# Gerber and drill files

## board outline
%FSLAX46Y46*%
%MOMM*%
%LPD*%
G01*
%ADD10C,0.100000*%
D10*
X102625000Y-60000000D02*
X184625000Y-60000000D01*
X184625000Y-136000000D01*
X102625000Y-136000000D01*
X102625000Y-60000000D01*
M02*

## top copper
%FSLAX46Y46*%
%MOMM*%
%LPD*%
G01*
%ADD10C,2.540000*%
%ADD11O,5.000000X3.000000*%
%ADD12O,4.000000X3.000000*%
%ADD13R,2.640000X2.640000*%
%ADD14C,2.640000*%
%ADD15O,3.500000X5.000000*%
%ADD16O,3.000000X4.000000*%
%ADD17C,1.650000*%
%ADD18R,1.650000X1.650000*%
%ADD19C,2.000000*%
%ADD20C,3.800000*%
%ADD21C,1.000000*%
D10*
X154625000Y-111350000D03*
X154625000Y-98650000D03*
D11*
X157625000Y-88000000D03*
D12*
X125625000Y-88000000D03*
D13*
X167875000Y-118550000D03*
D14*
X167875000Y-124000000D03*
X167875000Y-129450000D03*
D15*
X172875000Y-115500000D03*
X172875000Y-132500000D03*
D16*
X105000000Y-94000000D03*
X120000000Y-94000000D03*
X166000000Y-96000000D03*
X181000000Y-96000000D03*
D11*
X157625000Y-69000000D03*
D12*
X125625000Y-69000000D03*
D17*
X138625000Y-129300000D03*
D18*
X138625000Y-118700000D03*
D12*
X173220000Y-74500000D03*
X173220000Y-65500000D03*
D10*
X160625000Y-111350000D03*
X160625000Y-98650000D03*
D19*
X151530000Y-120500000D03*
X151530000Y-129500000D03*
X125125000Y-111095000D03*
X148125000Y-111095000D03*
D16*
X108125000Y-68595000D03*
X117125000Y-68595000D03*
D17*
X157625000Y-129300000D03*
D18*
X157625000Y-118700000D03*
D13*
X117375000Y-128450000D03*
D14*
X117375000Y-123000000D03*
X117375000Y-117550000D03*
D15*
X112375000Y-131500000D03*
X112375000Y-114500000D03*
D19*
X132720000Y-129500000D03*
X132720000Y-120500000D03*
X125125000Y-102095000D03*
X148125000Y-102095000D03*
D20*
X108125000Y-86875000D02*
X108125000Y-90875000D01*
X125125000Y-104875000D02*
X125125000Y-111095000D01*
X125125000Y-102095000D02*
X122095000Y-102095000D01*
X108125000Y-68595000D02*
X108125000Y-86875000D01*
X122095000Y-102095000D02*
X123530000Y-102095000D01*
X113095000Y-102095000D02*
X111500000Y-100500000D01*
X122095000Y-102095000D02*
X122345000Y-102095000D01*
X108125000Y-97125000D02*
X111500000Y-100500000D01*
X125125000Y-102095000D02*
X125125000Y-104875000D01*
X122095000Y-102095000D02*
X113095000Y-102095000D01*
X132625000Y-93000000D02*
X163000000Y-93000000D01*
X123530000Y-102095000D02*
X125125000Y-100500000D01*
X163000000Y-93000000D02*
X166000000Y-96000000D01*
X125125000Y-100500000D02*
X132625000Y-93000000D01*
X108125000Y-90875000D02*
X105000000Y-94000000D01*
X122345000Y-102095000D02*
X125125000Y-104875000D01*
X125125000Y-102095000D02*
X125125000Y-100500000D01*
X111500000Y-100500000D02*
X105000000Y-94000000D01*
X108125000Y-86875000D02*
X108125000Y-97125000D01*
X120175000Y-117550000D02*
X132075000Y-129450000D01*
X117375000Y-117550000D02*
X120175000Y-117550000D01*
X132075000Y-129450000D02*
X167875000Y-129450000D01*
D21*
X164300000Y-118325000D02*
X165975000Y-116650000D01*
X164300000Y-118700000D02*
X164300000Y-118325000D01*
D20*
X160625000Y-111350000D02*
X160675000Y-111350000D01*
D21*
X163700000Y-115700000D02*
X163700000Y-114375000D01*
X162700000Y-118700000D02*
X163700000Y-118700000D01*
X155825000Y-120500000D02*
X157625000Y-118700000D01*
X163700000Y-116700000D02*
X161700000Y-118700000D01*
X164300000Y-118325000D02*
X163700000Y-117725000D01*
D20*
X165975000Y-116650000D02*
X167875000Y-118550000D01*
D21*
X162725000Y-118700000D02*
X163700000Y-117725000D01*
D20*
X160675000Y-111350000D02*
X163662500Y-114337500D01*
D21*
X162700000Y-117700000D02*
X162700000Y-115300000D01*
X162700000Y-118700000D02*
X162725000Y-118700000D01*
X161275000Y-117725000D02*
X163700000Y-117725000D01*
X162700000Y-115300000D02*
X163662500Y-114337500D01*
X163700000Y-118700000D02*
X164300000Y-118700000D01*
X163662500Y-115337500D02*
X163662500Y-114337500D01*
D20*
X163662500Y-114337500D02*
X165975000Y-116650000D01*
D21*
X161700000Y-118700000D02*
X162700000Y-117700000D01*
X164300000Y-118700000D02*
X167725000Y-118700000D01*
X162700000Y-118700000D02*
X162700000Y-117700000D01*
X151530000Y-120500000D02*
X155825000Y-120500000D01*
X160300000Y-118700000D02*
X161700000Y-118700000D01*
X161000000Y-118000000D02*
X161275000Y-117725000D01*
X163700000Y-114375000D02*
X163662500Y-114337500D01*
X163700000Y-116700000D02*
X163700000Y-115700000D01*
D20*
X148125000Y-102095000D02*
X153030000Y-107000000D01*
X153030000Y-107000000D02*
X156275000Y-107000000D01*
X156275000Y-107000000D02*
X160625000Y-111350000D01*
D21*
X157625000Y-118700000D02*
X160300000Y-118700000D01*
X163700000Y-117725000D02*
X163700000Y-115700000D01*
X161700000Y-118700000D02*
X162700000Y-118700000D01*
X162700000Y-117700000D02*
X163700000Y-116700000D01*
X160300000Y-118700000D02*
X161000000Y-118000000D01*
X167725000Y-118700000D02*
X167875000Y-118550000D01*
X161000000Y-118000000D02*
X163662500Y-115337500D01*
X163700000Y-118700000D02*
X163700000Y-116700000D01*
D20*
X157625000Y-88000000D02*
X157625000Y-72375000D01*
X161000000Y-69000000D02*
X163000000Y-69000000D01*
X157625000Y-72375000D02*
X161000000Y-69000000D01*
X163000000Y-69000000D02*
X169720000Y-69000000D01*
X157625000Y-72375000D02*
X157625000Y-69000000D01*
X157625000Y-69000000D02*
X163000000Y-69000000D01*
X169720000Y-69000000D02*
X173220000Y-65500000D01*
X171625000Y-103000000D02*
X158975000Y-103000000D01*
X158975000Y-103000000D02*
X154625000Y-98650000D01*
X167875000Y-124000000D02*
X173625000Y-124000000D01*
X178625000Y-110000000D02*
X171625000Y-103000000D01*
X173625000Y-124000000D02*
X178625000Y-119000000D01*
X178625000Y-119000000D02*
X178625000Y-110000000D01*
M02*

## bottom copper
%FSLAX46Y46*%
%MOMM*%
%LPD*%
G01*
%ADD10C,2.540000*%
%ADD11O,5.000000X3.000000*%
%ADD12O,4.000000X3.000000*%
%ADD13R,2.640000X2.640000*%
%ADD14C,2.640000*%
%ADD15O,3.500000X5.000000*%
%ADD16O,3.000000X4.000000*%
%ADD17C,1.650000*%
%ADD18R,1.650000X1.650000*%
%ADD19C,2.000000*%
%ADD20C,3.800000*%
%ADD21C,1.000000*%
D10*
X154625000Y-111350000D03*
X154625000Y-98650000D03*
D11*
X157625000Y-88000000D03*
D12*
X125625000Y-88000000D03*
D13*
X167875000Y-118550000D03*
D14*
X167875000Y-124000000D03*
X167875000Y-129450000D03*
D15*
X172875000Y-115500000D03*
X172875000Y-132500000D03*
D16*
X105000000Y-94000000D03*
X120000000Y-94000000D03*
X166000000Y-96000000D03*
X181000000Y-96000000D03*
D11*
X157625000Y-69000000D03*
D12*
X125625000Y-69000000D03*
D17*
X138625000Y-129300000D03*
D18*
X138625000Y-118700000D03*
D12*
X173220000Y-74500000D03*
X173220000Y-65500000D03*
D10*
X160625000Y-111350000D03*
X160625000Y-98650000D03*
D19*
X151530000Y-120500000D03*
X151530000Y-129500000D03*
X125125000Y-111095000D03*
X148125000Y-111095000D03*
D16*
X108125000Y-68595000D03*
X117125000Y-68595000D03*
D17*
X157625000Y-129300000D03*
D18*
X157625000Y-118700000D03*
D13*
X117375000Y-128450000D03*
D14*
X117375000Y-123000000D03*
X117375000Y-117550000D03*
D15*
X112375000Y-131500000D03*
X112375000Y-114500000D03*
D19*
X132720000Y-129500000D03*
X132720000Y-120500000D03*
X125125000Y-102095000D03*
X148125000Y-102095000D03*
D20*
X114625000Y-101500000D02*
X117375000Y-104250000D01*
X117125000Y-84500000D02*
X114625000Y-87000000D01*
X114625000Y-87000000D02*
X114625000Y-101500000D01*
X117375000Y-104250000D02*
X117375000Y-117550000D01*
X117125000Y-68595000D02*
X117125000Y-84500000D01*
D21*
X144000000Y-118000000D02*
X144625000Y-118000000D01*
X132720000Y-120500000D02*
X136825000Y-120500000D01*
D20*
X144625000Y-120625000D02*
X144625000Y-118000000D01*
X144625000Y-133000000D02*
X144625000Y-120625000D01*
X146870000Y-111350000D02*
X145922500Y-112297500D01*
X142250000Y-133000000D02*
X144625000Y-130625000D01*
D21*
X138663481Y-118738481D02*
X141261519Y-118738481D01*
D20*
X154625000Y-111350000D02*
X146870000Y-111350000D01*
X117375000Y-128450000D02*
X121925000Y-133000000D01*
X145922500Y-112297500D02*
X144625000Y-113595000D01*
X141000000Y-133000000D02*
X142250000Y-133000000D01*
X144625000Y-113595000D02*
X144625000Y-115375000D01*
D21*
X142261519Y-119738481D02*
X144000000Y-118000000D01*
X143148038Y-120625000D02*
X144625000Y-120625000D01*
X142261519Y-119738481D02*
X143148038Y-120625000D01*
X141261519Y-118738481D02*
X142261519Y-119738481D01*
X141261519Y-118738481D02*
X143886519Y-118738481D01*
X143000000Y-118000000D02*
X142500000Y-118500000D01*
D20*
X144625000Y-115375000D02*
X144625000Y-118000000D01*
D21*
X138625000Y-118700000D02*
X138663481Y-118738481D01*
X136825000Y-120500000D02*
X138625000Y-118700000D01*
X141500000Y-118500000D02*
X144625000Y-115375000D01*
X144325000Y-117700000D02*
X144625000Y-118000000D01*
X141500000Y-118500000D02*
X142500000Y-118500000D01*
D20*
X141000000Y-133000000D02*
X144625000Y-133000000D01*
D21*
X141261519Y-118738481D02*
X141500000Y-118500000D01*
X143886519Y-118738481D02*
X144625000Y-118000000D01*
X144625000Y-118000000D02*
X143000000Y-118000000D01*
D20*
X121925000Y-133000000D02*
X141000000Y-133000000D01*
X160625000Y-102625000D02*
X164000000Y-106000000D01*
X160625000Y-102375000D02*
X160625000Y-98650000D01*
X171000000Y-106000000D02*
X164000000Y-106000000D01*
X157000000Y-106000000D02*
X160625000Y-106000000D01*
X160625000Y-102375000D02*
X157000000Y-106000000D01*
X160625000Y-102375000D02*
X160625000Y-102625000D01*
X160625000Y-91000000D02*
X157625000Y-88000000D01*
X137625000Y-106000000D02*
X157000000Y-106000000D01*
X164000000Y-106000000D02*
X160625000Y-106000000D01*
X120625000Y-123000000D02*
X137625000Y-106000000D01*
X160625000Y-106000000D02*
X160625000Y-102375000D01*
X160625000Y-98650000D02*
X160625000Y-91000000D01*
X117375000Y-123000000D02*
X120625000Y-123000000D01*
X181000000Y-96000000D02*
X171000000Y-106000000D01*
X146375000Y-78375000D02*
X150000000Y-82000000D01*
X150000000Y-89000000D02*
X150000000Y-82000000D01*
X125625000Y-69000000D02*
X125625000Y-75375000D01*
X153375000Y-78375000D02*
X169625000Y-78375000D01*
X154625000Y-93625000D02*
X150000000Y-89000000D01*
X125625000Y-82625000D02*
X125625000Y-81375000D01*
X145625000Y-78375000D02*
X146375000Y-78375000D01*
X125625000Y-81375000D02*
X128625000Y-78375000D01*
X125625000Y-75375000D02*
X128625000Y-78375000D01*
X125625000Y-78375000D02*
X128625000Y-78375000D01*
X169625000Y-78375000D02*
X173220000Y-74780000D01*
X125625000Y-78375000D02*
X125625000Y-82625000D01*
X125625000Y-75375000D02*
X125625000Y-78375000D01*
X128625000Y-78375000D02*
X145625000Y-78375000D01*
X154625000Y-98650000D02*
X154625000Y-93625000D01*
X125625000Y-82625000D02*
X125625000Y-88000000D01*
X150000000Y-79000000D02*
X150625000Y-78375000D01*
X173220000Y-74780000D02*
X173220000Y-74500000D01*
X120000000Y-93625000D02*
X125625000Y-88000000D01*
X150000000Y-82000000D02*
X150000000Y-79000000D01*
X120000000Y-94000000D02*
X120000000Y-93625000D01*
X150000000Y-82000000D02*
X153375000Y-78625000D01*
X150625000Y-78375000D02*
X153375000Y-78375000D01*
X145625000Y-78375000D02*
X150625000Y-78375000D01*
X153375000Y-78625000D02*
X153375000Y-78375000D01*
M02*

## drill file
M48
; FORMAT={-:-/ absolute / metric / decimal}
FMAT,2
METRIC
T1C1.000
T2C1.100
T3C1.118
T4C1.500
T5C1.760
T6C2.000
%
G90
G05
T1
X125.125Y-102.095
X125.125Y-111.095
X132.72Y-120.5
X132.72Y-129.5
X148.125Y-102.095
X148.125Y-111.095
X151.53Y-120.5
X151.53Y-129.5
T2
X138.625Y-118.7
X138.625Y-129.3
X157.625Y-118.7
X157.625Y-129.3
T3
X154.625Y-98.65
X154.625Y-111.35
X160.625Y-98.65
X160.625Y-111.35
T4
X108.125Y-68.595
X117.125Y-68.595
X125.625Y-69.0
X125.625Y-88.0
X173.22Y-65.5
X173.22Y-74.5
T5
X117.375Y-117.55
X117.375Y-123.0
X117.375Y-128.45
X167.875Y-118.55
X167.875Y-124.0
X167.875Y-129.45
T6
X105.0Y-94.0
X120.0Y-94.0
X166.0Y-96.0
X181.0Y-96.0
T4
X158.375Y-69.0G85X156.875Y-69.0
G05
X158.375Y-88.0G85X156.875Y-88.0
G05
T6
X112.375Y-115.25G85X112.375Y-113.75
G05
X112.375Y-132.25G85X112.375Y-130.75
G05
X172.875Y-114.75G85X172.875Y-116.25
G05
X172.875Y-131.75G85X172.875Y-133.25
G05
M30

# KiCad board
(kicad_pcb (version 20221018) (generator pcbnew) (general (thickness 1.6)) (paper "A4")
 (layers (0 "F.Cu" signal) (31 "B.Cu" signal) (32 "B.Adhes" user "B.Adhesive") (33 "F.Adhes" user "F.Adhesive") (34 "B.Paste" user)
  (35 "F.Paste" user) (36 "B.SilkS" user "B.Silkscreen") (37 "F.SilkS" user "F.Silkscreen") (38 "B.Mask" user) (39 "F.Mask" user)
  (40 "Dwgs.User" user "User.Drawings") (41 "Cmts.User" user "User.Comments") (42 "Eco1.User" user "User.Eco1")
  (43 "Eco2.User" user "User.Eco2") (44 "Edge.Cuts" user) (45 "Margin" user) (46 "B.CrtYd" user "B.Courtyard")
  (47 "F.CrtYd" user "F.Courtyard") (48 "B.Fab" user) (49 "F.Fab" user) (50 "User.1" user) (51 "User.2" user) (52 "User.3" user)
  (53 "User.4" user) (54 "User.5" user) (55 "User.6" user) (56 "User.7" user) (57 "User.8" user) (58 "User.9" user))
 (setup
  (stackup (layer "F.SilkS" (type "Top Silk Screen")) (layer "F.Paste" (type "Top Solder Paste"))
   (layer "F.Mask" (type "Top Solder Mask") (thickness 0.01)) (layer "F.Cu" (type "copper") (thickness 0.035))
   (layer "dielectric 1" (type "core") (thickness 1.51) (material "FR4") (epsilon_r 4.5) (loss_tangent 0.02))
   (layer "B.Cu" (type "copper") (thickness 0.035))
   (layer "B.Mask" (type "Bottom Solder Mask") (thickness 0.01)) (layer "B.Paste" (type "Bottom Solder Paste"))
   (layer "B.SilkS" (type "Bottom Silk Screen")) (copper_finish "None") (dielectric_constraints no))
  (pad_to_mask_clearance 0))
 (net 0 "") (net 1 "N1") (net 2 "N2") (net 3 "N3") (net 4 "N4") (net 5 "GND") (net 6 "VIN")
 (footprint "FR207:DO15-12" (layer "F.Cu") (at 154.625 105 -90)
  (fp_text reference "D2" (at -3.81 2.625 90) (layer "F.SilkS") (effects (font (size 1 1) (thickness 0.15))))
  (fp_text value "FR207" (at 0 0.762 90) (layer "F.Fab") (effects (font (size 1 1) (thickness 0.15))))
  (pad "A" thru_hole circle (at 6.35 0 270) (size 2.54 2.54) (drill 1.1176) (layers "*.Cu" "*.Mask") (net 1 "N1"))
  (pad "C" thru_hole circle (at -6.35 0 270) (size 2.54 2.54) (drill 1.1176) (layers "*.Cu" "*.Mask") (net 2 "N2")))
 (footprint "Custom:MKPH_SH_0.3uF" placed (layer "F.Cu") (at 141.625 100 180)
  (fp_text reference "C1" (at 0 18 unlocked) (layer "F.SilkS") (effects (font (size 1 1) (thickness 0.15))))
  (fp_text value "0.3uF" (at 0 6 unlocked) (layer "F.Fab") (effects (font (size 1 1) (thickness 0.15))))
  (pad "1" thru_hole oval (at -16 12 180) (size 5 3) (drill oval 3 1.5) (layers "*.Cu" "*.Mask") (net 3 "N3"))
  (pad "2" thru_hole oval (at 16 12 180) (size 4 3) (drill 1.5) (layers "*.Cu" "*.Mask") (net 2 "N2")))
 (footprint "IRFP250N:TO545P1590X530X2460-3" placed (layer "F.Cu") (at 167.875 124 -90)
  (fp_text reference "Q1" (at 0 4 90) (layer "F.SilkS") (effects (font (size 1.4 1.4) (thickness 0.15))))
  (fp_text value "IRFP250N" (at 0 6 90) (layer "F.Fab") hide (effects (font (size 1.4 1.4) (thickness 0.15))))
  (pad "1" thru_hole rect (at -5.45 0 270) (size 2.64 2.64) (drill 1.76) (layers "*.Cu" "*.Mask") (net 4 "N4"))
  (pad "2" thru_hole circle (at 0 0 270) (size 2.64 2.64) (drill 1.76) (layers "*.Cu" "*.Mask") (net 2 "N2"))
  (pad "3" thru_hole circle (at 5.45 0 270) (size 2.64 2.64) (drill 1.76) (layers "*.Cu" "*.Mask") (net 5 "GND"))
  (pad "4" thru_hole oval (at -8.5 -5 270) (size 5 3.5) (drill oval 3.5 2) (layers "*.Cu" "*.Mask"))
  (pad "5" thru_hole oval (at 8.5 -5 270) (size 5 3.5) (drill oval 3.5 2) (layers "*.Cu" "*.Mask")))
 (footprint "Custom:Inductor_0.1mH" (layer "F.Cu") (at 100 94 90)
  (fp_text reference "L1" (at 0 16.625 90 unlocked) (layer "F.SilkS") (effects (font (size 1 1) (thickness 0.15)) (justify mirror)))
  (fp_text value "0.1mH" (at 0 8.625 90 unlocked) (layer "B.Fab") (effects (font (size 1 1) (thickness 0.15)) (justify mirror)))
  (pad "1" thru_hole oval (at 0 5 90) (size 4 3) (drill 2) (layers "*.Cu" "*.Mask") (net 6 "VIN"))
  (pad "2" thru_hole oval (at 0 20 90) (size 4 3) (drill 2) (layers "*.Cu" "*.Mask") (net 2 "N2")))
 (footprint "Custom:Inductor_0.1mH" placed (layer "F.Cu") (at 161 96 90)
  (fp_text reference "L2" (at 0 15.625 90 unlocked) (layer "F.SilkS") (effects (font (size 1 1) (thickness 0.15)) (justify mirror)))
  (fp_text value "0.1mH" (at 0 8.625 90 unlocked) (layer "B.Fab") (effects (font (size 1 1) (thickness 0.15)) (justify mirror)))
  (pad "1" thru_hole oval (at 0 5 90) (size 4 3) (drill 2) (layers "*.Cu" "*.Mask") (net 6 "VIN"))
  (pad "2" thru_hole oval (at 0 20 90) (size 4 3) (drill 2) (layers "*.Cu" "*.Mask") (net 3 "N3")))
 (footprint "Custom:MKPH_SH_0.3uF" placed (layer "F.Cu") (at 141.625 81 180)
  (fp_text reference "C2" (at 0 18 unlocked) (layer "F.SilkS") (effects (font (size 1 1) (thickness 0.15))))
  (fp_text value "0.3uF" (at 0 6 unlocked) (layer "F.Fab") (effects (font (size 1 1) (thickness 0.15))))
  (pad "1" thru_hole oval (at -16 12 180) (size 5 3) (drill oval 3 1.5) (layers "*.Cu" "*.Mask") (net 3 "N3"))
  (pad "2" thru_hole oval (at 16 12 180) (size 4 3) (drill 1.5) (layers "*.Cu" "*.Mask") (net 2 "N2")))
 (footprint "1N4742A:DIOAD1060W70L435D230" (layer "F.Cu") (at 138.625 124 -90)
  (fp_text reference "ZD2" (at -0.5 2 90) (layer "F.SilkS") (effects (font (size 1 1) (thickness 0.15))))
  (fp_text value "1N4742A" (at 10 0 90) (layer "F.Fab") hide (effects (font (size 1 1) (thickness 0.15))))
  (pad "A" thru_hole circle (at 5.3 0 270) (size 1.65 1.65) (drill 1.1) (layers "*.Cu" "*.Mask") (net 5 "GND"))
  (pad "C" thru_hole rect (at -5.3 0 270) (size 1.65 1.65) (drill 1.1) (layers "*.Cu" "*.Mask") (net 1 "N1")))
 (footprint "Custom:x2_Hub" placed (layer "F.Cu") (at 161.22 69.5 90)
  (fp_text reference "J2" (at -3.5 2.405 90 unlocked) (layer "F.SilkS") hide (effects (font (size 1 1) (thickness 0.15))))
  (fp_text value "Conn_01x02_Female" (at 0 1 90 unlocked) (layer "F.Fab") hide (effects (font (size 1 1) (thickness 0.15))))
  (pad "1" thru_hole oval (at -5 12 90) (size 3 4) (drill 1.5) (layers "*.Cu" "*.Mask") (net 2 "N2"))
  (pad "2" thru_hole oval (at 4 12 90) (size 3 4) (drill 1.5) (layers "*.Cu" "*.Mask") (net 3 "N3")))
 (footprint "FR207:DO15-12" (layer "F.Cu") (at 160.625 105 -90)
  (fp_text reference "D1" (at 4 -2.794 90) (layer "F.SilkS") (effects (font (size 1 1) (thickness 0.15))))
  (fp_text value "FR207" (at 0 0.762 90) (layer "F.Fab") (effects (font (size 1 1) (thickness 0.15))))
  (pad "A" thru_hole circle (at 6.35 0 270) (size 2.54 2.54) (drill 1.1176) (layers "*.Cu" "*.Mask") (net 4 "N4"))
  (pad "C" thru_hole circle (at -6.35 0 270) (size 2.54 2.54) (drill 1.1176) (layers "*.Cu" "*.Mask") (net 3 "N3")))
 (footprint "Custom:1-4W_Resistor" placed (layer "F.Cu") (at 156.53 125.5 -90)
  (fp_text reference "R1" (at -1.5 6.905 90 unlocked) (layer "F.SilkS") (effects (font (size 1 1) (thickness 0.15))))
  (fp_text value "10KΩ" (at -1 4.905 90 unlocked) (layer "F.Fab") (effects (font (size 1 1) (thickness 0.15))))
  (pad "1" thru_hole circle (at -5 5 270) (size 2 2) (drill 1) (layers "*.Cu" "*.Mask") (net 4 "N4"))
  (pad "2" thru_hole circle (at 4 5 270) (size 2 2) (drill 1) (layers "*.Cu" "*.Mask") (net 5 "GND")))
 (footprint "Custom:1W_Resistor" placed (layer "F.Cu") (at 136.125 104.095)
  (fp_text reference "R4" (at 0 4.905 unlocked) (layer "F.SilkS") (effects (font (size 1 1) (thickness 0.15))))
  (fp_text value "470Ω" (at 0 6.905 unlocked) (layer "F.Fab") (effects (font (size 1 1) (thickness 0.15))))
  (pad "1" thru_hole circle (at -11 7) (size 2 2) (drill 1) (layers "*.Cu" "*.Mask") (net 6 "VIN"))
  (pad "2" thru_hole circle (at 12 7) (size 2 2) (drill 1) (layers "*.Cu" "*.Mask") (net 1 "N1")))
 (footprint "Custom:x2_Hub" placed (layer "F.Cu") (at 113.125 56.595)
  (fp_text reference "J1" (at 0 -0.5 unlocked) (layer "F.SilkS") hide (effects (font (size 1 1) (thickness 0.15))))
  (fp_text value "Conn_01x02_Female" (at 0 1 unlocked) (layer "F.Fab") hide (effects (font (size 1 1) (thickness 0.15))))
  (pad "1" thru_hole oval (at -5 12) (size 3 4) (drill 1.5) (layers "*.Cu" "*.Mask") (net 6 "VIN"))
  (pad "2" thru_hole oval (at 4 12) (size 3 4) (drill 1.5) (layers "*.Cu" "*.Mask") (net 5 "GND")))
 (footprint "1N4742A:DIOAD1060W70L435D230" (layer "F.Cu") (at 157.625 124 -90)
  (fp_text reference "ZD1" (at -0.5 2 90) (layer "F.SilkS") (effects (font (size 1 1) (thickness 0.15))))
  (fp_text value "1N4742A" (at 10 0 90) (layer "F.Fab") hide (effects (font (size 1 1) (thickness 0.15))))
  (pad "A" thru_hole circle (at 5.3 0 270) (size 1.65 1.65) (drill 1.1) (layers "*.Cu" "*.Mask") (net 5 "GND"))
  (pad "C" thru_hole rect (at -5.3 0 270) (size 1.65 1.65) (drill 1.1) (layers "*.Cu" "*.Mask") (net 4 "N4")))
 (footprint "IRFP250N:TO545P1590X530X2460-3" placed (layer "F.Cu") (at 117.375 123 90)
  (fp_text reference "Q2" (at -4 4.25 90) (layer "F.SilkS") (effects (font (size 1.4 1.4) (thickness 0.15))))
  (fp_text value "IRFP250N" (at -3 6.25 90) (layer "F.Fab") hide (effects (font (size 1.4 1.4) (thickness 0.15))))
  (pad "1" thru_hole rect (at -5.45 0 90) (size 2.64 2.64) (drill 1.76) (layers "*.Cu" "*.Mask") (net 1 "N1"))
  (pad "2" thru_hole circle (at 0 0 90) (size 2.64 2.64) (drill 1.76) (layers "*.Cu" "*.Mask") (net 3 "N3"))
  (pad "3" thru_hole circle (at 5.45 0 90) (size 2.64 2.64) (drill 1.76) (layers "*.Cu" "*.Mask") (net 5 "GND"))
  (pad "4" thru_hole oval (at -8.5 -5 90) (size 5 3.5) (drill oval 3.5 2) (layers "*.Cu" "*.Mask"))
  (pad "5" thru_hole oval (at 8.5 -5 90) (size 5 3.5) (drill oval 3.5 2) (layers "*.Cu" "*.Mask")))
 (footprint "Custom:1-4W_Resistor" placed (layer "F.Cu") (at 127.72 124.5 90)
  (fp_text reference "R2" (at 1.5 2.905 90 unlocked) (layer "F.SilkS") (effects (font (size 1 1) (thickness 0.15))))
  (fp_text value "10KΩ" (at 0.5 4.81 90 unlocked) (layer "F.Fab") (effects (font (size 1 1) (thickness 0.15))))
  (pad "1" thru_hole circle (at -5 5 90) (size 2 2) (drill 1) (layers "*.Cu" "*.Mask") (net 5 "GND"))
  (pad "2" thru_hole circle (at 4 5 90) (size 2 2) (drill 1) (layers "*.Cu" "*.Mask") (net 1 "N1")))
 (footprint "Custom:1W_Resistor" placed (layer "F.Cu") (at 136.125 95.095)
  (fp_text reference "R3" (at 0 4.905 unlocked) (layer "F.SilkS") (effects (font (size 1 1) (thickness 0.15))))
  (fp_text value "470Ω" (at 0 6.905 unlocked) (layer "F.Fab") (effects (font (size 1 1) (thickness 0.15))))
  (pad "1" thru_hole circle (at -11 7) (size 2 2) (drill 1) (layers "*.Cu" "*.Mask") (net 6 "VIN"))
  (pad "2" thru_hole circle (at 12 7) (size 2 2) (drill 1) (layers "*.Cu" "*.Mask") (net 4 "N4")))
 (gr_rect (start 102.625 60) (end 184.625 136) (stroke (width 0.1) (type solid)) (fill none) (layer "Edge.Cuts"))
 (segment (start 108.125 86.875) (end 108.125 90.875) (width 3.8) (layer "F.Cu") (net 6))
 (segment (start 125.125 104.875) (end 125.125 111.095) (width 3.8) (layer "F.Cu") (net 6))
 (segment (start 125.125 102.095) (end 122.095 102.095) (width 3.8) (layer "F.Cu") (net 6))
 (segment (start 108.125 68.595) (end 108.125 86.875) (width 3.8) (layer "F.Cu") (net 6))
 (segment (start 122.095 102.095) (end 123.53 102.095) (width 3.8) (layer "F.Cu") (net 6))
 (segment (start 113.095 102.095) (end 111.5 100.5) (width 3.8) (layer "F.Cu") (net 6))
 (segment (start 122.095 102.095) (end 122.345 102.095) (width 3.8) (layer "F.Cu") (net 6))
 (segment (start 108.125 97.125) (end 111.5 100.5) (width 3.8) (layer "F.Cu") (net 6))
 (segment (start 125.125 102.095) (end 125.125 104.875) (width 3.8) (layer "F.Cu") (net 6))
 (segment (start 122.095 102.095) (end 113.095 102.095) (width 3.8) (layer "F.Cu") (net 6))
 (segment (start 132.625 93) (end 163 93) (width 3.8) (layer "F.Cu") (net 6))
 (segment (start 123.53 102.095) (end 125.125 100.5) (width 3.8) (layer "F.Cu") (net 6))
 (segment (start 163 93) (end 166 96) (width 3.8) (layer "F.Cu") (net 6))
 (segment (start 125.125 100.5) (end 132.625 93) (width 3.8) (layer "F.Cu") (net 6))
 (segment (start 108.125 90.875) (end 105 94) (width 3.8) (layer "F.Cu") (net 6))
 (segment (start 122.345 102.095) (end 125.125 104.875) (width 3.8) (layer "F.Cu") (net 6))
 (segment (start 125.125 102.095) (end 125.125 100.5) (width 3.8) (layer "F.Cu") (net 6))
 (segment (start 111.5 100.5) (end 105 94) (width 3.8) (layer "F.Cu") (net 6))
 (segment (start 108.125 86.875) (end 108.125 97.125) (width 3.8) (layer "F.Cu") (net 6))
 (segment (start 120.175 117.55) (end 132.075 129.45) (width 3.8) (layer "F.Cu") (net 5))
 (segment (start 117.375 117.55) (end 120.175 117.55) (width 3.8) (layer "F.Cu") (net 5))
 (segment (start 132.075 129.45) (end 167.875 129.45) (width 3.8) (layer "F.Cu") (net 5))
 (segment (start 114.625 101.5) (end 117.375 104.25) (width 3.8) (layer "B.Cu") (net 5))
 (segment (start 117.125 84.5) (end 114.625 87) (width 3.8) (layer "B.Cu") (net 5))
 (segment (start 114.625 87) (end 114.625 101.5) (width 3.8) (layer "B.Cu") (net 5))
 (segment (start 117.375 104.25) (end 117.375 117.55) (width 3.8) (layer "B.Cu") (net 5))
 (segment (start 117.125 68.595) (end 117.125 84.5) (width 3.8) (layer "B.Cu") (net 5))
 (segment (start 164.3 118.325) (end 165.975 116.65) (width 1) (layer "F.Cu") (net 4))
 (segment (start 164.3 118.7) (end 164.3 118.325) (width 1) (layer "F.Cu") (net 4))
 (segment (start 160.625 111.35) (end 160.675 111.35) (width 3.8) (layer "F.Cu") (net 4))
 (segment (start 163.7 115.7) (end 163.7 114.375) (width 1) (layer "F.Cu") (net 4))
 (segment (start 162.7 118.7) (end 163.7 118.7) (width 1) (layer "F.Cu") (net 4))
 (segment (start 155.825 120.5) (end 157.625 118.7) (width 1) (layer "F.Cu") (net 4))
 (segment (start 163.7 116.7) (end 161.7 118.7) (width 1) (layer "F.Cu") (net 4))
 (segment (start 164.3 118.325) (end 163.7 117.725) (width 1) (layer "F.Cu") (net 4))
 (segment (start 165.975 116.65) (end 167.875 118.55) (width 3.8) (layer "F.Cu") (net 4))
 (segment (start 162.725 118.7) (end 163.7 117.725) (width 1) (layer "F.Cu") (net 4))
 (segment (start 160.675 111.35) (end 163.6625 114.3375) (width 3.8) (layer "F.Cu") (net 4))
 (segment (start 162.7 117.7) (end 162.7 115.3) (width 1) (layer "F.Cu") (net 4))
 (segment (start 162.7 118.7) (end 162.725 118.7) (width 1) (layer "F.Cu") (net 4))
 (segment (start 161.275 117.725) (end 163.7 117.725) (width 1) (layer "F.Cu") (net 4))
 (segment (start 162.7 115.3) (end 163.6625 114.3375) (width 1) (layer "F.Cu") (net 4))
 (segment (start 163.7 118.7) (end 164.3 118.7) (width 1) (layer "F.Cu") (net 4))
 (segment (start 163.6625 115.3375) (end 163.6625 114.3375) (width 1) (layer "F.Cu") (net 4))
 (segment (start 163.6625 114.3375) (end 165.975 116.65) (width 3.8) (layer "F.Cu") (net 4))
 (segment (start 161.7 118.7) (end 162.7 117.7) (width 1) (layer "F.Cu") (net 4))
 (segment (start 164.3 118.7) (end 167.725 118.7) (width 1) (layer "F.Cu") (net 4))
 (segment (start 162.7 118.7) (end 162.7 117.7) (width 1) (layer "F.Cu") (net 4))
 (segment (start 151.53 120.5) (end 155.825 120.5) (width 1) (layer "F.Cu") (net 4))
 (segment (start 160.3 118.7) (end 161.7 118.7) (width 1) (layer "F.Cu") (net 4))
 (segment (start 161 118) (end 161.275 117.725) (width 1) (layer "F.Cu") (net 4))
 (segment (start 163.7 114.375) (end 163.6625 114.3375) (width 1) (layer "F.Cu") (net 4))
 (segment (start 163.7 116.7) (end 163.7 115.7) (width 1) (layer "F.Cu") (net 4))
 (segment (start 148.125 102.095) (end 153.03 107) (width 3.8) (layer "F.Cu") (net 4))
 (segment (start 153.03 107) (end 156.275 107) (width 3.8) (layer "F.Cu") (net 4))
 (segment (start 156.275 107) (end 160.625 111.35) (width 3.8) (layer "F.Cu") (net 4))
 (segment (start 157.625 118.7) (end 160.3 118.7) (width 1) (layer "F.Cu") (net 4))
 (segment (start 163.7 117.725) (end 163.7 115.7) (width 1) (layer "F.Cu") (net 4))
 (segment (start 161.7 118.7) (end 162.7 118.7) (width 1) (layer "F.Cu") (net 4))
 (segment (start 162.7 117.7) (end 163.7 116.7) (width 1) (layer "F.Cu") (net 4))
 (segment (start 160.3 118.7) (end 161 118) (width 1) (layer "F.Cu") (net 4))
 (segment (start 167.725 118.7) (end 167.875 118.55) (width 1) (layer "F.Cu") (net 4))
 (segment (start 161 118) (end 163.6625 115.3375) (width 1) (layer "F.Cu") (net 4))
 (segment (start 163.7 118.7) (end 163.7 116.7) (width 1) (layer "F.Cu") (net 4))
 (segment (start 144 118) (end 144.625 118) (width 1) (layer "B.Cu") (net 1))
 (segment (start 132.72 120.5) (end 136.825 120.5) (width 1) (layer "B.Cu") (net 1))
 (segment (start 144.625 120.625) (end 144.625 118) (width 3.8) (layer "B.Cu") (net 1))
 (segment (start 144.625 133) (end 144.625 120.625) (width 3.8) (layer "B.Cu") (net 1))
 (segment (start 146.87 111.35) (end 145.9225 112.2975) (width 3.8) (layer "B.Cu") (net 1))
 (segment (start 142.25 133) (end 144.625 130.625) (width 3.8) (layer "B.Cu") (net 1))
 (segment (start 138.663481 118.738481) (end 141.261519 118.738481) (width 1) (layer "B.Cu") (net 1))
 (segment (start 154.625 111.35) (end 146.87 111.35) (width 3.8) (layer "B.Cu") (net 1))
 (segment (start 117.375 128.45) (end 121.925 133) (width 3.8) (layer "B.Cu") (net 1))
 (segment (start 145.9225 112.2975) (end 144.625 113.595) (width 3.8) (layer "B.Cu") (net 1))
 (segment (start 141 133) (end 142.25 133) (width 3.8) (layer "B.Cu") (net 1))
 (segment (start 144.625 113.595) (end 144.625 115.375) (width 3.8) (layer "B.Cu") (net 1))
 (segment (start 142.261519 119.738481) (end 144 118) (width 1) (layer "B.Cu") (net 1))
 (segment (start 143.148038 120.625) (end 144.625 120.625) (width 1) (layer "B.Cu") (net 1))
 (segment (start 142.261519 119.738481) (end 143.148038 120.625) (width 1) (layer "B.Cu") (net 1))
 (segment (start 141.261519 118.738481) (end 142.261519 119.738481) (width 1) (layer "B.Cu") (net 1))
 (segment (start 141.261519 118.738481) (end 143.886519 118.738481) (width 1) (layer "B.Cu") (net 1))
 (segment (start 143 118) (end 142.5 118.5) (width 1) (layer "B.Cu") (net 1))
 (segment (start 144.625 115.375) (end 144.625 118) (width 3.8) (layer "B.Cu") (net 1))
 (segment (start 138.625 118.7) (end 138.663481 118.738481) (width 1) (layer "B.Cu") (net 1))
 (segment (start 136.825 120.5) (end 138.625 118.7) (width 1) (layer "B.Cu") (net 1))
 (segment (start 141.5 118.5) (end 144.625 115.375) (width 1) (layer "B.Cu") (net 1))
 (segment (start 144.325 117.7) (end 144.625 118) (width 1) (layer "B.Cu") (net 1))
 (segment (start 141.5 118.5) (end 142.5 118.5) (width 1) (layer "B.Cu") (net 1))
 (segment (start 141 133) (end 144.625 133) (width 3.8) (layer "B.Cu") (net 1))
 (segment (start 141.261519 118.738481) (end 141.5 118.5) (width 1) (layer "B.Cu") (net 1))
 (segment (start 143.886519 118.738481) (end 144.625 118) (width 1) (layer "B.Cu") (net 1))
 (segment (start 144.625 118) (end 143 118) (width 1) (layer "B.Cu") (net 1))
 (segment (start 121.925 133) (end 141 133) (width 3.8) (layer "B.Cu") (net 1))
 (segment (start 157.625 88) (end 157.625 72.375) (width 3.8) (layer "F.Cu") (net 3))
 (segment (start 161 69) (end 163 69) (width 3.8) (layer "F.Cu") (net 3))
 (segment (start 157.625 72.375) (end 161 69) (width 3.8) (layer "F.Cu") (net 3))
 (segment (start 163 69) (end 169.72 69) (width 3.8) (layer "F.Cu") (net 3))
 (segment (start 157.625 72.375) (end 157.625 69) (width 3.8) (layer "F.Cu") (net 3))
 (segment (start 157.625 69) (end 163 69) (width 3.8) (layer "F.Cu") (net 3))
 (segment (start 169.72 69) (end 173.22 65.5) (width 3.8) (layer "F.Cu") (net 3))
 (segment (start 160.625 102.625) (end 164 106) (width 3.8) (layer "B.Cu") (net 3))
 (segment (start 160.625 102.375) (end 160.625 98.65) (width 3.8) (layer "B.Cu") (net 3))
 (segment (start 171 106) (end 164 106) (width 3.8) (layer "B.Cu") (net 3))
 (segment (start 157 106) (end 160.625 106) (width 3.8) (layer "B.Cu") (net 3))
 (segment (start 160.625 102.375) (end 157 106) (width 3.8) (layer "B.Cu") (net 3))
 (segment (start 160.625 102.375) (end 160.625 102.625) (width 3.8) (layer "B.Cu") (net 3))
 (segment (start 160.625 91) (end 157.625 88) (width 3.8) (layer "B.Cu") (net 3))
 (segment (start 137.625 106) (end 157 106) (width 3.8) (layer "B.Cu") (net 3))
 (segment (start 164 106) (end 160.625 106) (width 3.8) (layer "B.Cu") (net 3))
 (segment (start 120.625 123) (end 137.625 106) (width 3.8) (layer "B.Cu") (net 3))
 (segment (start 160.625 106) (end 160.625 102.375) (width 3.8) (layer "B.Cu") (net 3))
 (segment (start 160.625 98.65) (end 160.625 91) (width 3.8) (layer "B.Cu") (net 3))
 (segment (start 117.375 123) (end 120.625 123) (width 3.8) (layer "B.Cu") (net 3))
 (segment (start 181 96) (end 171 106) (width 3.8) (layer "B.Cu") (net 3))
 (segment (start 171.625 103) (end 158.975 103) (width 3.8) (layer "F.Cu") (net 2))
 (segment (start 158.975 103) (end 154.625 98.65) (width 3.8) (layer "F.Cu") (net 2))
 (segment (start 167.875 124) (end 173.625 124) (width 3.8) (layer "F.Cu") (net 2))
 (segment (start 178.625 110) (end 171.625 103) (width 3.8) (layer "F.Cu") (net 2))
 (segment (start 173.625 124) (end 178.625 119) (width 3.8) (layer "F.Cu") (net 2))
 (segment (start 178.625 119) (end 178.625 110) (width 3.8) (layer "F.Cu") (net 2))
 (segment (start 146.375 78.375) (end 150 82) (width 3.8) (layer "B.Cu") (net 2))
 (segment (start 150 89) (end 150 82) (width 3.8) (layer "B.Cu") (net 2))
 (segment (start 125.625 69) (end 125.625 75.375) (width 3.8) (layer "B.Cu") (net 2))
 (segment (start 153.375 78.375) (end 169.625 78.375) (width 3.8) (layer "B.Cu") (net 2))
 (segment (start 154.625 93.625) (end 150 89) (width 3.8) (layer "B.Cu") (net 2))
 (segment (start 125.625 82.625) (end 125.625 81.375) (width 3.8) (layer "B.Cu") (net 2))
 (segment (start 145.625 78.375) (end 146.375 78.375) (width 3.8) (layer "B.Cu") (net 2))
 (segment (start 125.625 81.375) (end 128.625 78.375) (width 3.8) (layer "B.Cu") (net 2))
 (segment (start 125.625 75.375) (end 128.625 78.375) (width 3.8) (layer "B.Cu") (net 2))
 (segment (start 125.625 78.375) (end 128.625 78.375) (width 3.8) (layer "B.Cu") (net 2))
 (segment (start 169.625 78.375) (end 173.22 74.78) (width 3.8) (layer "B.Cu") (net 2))
 (segment (start 125.625 78.375) (end 125.625 82.625) (width 3.8) (layer "B.Cu") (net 2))
 (segment (start 125.625 75.375) (end 125.625 78.375) (width 3.8) (layer "B.Cu") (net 2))
 (segment (start 128.625 78.375) (end 145.625 78.375) (width 3.8) (layer "B.Cu") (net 2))
 (segment (start 154.625 98.65) (end 154.625 93.625) (width 3.8) (layer "B.Cu") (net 2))
 (segment (start 125.625 82.625) (end 125.625 88) (width 3.8) (layer "B.Cu") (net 2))
 (segment (start 150 79) (end 150.625 78.375) (width 3.8) (layer "B.Cu") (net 2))
 (segment (start 173.22 74.78) (end 173.22 74.5) (width 3.8) (layer "B.Cu") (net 2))
 (segment (start 120 93.625) (end 125.625 88) (width 3.8) (layer "B.Cu") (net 2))
 (segment (start 150 82) (end 150 79) (width 3.8) (layer "B.Cu") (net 2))
 (segment (start 120 94) (end 120 93.625) (width 3.8) (layer "B.Cu") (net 2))
 (segment (start 150 82) (end 153.375 78.625) (width 3.8) (layer "B.Cu") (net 2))
 (segment (start 150.625 78.375) (end 153.375 78.375) (width 3.8) (layer "B.Cu") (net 2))
 (segment (start 145.625 78.375) (end 150.625 78.375) (width 3.8) (layer "B.Cu") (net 2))
 (segment (start 153.375 78.625) (end 153.375 78.375) (width 3.8) (layer "B.Cu") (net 2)))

